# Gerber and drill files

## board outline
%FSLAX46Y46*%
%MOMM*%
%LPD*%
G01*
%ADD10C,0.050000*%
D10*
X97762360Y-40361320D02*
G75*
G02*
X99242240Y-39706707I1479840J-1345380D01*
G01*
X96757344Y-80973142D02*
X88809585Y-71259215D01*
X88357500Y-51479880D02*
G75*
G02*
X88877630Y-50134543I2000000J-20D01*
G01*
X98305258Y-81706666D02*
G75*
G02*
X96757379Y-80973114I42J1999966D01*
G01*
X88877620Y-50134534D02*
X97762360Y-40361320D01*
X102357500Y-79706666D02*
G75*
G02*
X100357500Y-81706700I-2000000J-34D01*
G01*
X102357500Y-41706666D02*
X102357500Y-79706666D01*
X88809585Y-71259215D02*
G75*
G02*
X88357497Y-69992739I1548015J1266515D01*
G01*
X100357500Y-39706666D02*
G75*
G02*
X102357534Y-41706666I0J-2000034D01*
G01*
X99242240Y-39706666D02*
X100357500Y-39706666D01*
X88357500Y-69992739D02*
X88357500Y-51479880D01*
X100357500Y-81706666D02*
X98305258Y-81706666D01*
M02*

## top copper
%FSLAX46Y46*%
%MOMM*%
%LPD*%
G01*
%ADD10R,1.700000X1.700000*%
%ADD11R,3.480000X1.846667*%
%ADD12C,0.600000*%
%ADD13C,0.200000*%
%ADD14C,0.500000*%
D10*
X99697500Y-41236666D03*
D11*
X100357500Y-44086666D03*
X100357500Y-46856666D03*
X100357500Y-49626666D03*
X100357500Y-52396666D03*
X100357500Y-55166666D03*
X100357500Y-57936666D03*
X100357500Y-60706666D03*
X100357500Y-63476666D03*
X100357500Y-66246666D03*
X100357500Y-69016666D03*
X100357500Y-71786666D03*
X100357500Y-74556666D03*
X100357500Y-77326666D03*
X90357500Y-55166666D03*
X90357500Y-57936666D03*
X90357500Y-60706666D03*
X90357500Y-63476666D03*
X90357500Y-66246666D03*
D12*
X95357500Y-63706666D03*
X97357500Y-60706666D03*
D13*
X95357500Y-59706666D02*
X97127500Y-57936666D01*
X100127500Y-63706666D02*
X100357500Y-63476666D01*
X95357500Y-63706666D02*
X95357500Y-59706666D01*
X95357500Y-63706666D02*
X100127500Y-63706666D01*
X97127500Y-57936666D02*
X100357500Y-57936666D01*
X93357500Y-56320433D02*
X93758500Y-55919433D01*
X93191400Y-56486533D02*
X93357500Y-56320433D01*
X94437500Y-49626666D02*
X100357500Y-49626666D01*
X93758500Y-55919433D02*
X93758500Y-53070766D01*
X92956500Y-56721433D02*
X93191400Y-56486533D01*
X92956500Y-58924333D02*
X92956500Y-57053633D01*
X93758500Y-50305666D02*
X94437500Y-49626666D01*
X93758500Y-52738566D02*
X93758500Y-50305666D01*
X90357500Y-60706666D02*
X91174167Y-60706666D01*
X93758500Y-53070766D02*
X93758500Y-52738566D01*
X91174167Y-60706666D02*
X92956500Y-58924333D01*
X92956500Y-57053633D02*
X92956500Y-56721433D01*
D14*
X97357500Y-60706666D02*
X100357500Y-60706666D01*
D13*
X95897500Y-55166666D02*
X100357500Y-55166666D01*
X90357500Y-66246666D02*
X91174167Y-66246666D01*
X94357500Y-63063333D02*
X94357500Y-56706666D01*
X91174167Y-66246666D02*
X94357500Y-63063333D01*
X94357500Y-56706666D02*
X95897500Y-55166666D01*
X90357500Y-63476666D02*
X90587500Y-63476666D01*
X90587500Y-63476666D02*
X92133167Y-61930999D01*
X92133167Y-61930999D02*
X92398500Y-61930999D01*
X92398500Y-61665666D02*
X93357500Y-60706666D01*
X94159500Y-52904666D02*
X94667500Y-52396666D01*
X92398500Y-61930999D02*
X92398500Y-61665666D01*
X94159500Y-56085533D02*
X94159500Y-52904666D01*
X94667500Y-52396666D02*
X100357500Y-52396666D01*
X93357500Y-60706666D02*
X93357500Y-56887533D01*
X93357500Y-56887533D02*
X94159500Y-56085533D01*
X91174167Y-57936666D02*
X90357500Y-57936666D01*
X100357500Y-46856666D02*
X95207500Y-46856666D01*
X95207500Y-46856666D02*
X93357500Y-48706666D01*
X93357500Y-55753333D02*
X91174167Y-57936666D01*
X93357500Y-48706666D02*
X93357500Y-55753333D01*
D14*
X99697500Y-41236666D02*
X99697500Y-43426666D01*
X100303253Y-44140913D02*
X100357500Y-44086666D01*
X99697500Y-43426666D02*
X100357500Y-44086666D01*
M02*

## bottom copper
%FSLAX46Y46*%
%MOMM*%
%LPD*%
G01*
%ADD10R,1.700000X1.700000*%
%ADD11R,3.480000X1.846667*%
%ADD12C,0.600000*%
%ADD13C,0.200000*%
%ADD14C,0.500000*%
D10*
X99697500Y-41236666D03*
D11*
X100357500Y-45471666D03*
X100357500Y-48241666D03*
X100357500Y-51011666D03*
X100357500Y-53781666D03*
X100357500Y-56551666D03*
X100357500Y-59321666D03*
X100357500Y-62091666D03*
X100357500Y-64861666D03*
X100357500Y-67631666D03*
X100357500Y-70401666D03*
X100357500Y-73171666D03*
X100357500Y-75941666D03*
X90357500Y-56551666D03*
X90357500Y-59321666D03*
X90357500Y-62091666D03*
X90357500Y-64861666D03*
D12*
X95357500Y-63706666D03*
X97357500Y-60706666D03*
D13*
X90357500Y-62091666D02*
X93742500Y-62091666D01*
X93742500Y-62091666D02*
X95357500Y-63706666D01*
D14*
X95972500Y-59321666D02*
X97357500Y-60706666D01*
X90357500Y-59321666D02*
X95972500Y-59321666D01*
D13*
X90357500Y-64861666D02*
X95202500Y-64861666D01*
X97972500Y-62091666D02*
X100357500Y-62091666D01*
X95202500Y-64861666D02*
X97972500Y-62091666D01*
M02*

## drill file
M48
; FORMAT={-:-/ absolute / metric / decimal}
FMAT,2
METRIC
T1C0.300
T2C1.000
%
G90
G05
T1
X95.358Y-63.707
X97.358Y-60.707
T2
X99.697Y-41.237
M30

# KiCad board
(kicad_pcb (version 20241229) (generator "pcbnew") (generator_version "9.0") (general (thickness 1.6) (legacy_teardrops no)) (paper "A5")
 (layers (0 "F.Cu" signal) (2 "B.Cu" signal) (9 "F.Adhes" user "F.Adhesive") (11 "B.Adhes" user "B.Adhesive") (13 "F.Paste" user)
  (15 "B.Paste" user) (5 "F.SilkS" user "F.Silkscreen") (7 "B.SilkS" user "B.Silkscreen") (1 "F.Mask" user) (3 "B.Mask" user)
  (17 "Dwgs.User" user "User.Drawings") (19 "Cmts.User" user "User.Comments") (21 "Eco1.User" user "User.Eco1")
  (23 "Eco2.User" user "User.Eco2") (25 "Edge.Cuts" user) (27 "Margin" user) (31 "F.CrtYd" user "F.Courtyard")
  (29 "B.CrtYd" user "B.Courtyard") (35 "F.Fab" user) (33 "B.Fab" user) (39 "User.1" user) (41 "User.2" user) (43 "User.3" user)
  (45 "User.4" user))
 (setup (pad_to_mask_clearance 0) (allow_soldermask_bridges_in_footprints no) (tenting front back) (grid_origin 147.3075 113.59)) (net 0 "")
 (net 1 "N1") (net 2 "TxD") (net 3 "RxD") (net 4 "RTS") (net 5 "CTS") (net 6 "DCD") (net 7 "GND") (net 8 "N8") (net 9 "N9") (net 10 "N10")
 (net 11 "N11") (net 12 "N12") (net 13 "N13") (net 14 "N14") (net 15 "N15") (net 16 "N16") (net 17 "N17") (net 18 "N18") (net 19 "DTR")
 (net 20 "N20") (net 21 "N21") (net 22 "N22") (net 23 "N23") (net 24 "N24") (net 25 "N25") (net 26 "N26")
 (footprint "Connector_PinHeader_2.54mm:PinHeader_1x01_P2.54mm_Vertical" (layer "F.Cu") (at 99.6975 41.236666)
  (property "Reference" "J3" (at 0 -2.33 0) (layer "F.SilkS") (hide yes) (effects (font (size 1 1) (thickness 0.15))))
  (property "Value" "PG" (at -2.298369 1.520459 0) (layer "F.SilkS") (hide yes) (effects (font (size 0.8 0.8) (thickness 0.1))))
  (pad "1" thru_hole rect (at 0 0) (size 1.7 1.7) (drill 1) (layers "*.Cu" "*.Mask") (remove_unused_layers no) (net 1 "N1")))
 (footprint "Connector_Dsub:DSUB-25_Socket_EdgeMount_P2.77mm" (layer "F.Cu") (at 100.3575 60.706666 90)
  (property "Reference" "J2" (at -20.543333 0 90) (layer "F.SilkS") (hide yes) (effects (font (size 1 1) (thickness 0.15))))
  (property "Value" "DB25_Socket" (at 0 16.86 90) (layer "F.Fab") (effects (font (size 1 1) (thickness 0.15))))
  (pad "1" smd rect (at 16.62 0 90) (size 1.846667 3.48) (layers "F.Cu" "F.Mask" "F.Paste") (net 1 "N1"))
  (pad "2" smd rect (at 13.85 0 90) (size 1.846667 3.48) (layers "F.Cu" "F.Mask" "F.Paste") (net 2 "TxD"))
  (pad "3" smd rect (at 11.08 0 90) (size 1.846667 3.48) (layers "F.Cu" "F.Mask" "F.Paste") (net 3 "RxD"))
  (pad "4" smd rect (at 8.31 0 90) (size 1.846667 3.48) (layers "F.Cu" "F.Mask" "F.Paste") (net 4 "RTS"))
  (pad "5" smd rect (at 5.54 0 90) (size 1.846667 3.48) (layers "F.Cu" "F.Mask" "F.Paste") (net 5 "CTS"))
  (pad "6" smd rect (at 2.77 0 90) (size 1.846667 3.48) (layers "F.Cu" "F.Mask" "F.Paste") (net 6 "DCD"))
  (pad "7" smd rect (at 0 0 90) (size 1.846667 3.48) (layers "F.Cu" "F.Mask" "F.Paste") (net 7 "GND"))
  (pad "8" smd rect (at -2.77 0 90) (size 1.846667 3.48) (layers "F.Cu" "F.Mask" "F.Paste") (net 6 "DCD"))
  (pad "9" smd rect (at -5.54 0 90) (size 1.846667 3.48) (layers "F.Cu" "F.Mask" "F.Paste") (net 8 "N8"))
  (pad "10" smd rect (at -8.31 0 90) (size 1.846667 3.48) (layers "F.Cu" "F.Mask" "F.Paste") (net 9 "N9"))
  (pad "11" smd rect (at -11.08 0 90) (size 1.846667 3.48) (layers "F.Cu" "F.Mask" "F.Paste") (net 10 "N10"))
  (pad "12" smd rect (at -13.85 0 90) (size 1.846667 3.48) (layers "F.Cu" "F.Mask" "F.Paste") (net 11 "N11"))
  (pad "13" smd rect (at -16.62 0 90) (size 1.846667 3.48) (layers "F.Cu" "F.Mask" "F.Paste") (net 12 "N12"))
  (pad "14" smd rect (at 15.235 0 90) (size 1.846667 3.48) (layers "B.Cu" "B.Mask" "B.Paste") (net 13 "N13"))
  (pad "15" smd rect (at 12.465 0 90) (size 1.846667 3.48) (layers "B.Cu" "B.Mask" "B.Paste") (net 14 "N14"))
  (pad "16" smd rect (at 9.695 0 90) (size 1.846667 3.48) (layers "B.Cu" "B.Mask" "B.Paste") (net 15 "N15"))
  (pad "17" smd rect (at 6.925 0 90) (size 1.846667 3.48) (layers "B.Cu" "B.Mask" "B.Paste") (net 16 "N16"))
  (pad "18" smd rect (at 4.155 0 90) (size 1.846667 3.48) (layers "B.Cu" "B.Mask" "B.Paste") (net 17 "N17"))
  (pad "19" smd rect (at 1.385 0 90) (size 1.846667 3.48) (layers "B.Cu" "B.Mask" "B.Paste") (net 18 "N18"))
  (pad "20" smd rect (at -1.385 0 90) (size 1.846667 3.48) (layers "B.Cu" "B.Mask" "B.Paste") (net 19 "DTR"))
  (pad "21" smd rect (at -4.155 0 90) (size 1.846667 3.48) (layers "B.Cu" "B.Mask" "B.Paste") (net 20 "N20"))
  (pad "22" smd rect (at -6.925 0 90) (size 1.846667 3.48) (layers "B.Cu" "B.Mask" "B.Paste") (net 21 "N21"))
  (pad "23" smd rect (at -9.695 0 90) (size 1.846667 3.48) (layers "B.Cu" "B.Mask" "B.Paste") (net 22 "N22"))
  (pad "24" smd rect (at -12.465 0 90) (size 1.846667 3.48) (layers "B.Cu" "B.Mask" "B.Paste") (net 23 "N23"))
  (pad "25" smd rect (at -15.235 0 90) (size 1.846667 3.48) (layers "B.Cu" "B.Mask" "B.Paste") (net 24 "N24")))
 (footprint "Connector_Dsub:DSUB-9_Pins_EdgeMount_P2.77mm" (layer "F.Cu") (at 90.3575 60.706666 -90)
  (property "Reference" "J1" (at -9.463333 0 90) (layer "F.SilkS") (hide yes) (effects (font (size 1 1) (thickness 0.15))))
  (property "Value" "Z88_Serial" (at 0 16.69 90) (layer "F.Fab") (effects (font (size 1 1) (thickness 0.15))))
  (pad "1" smd rect (at -5.54 0 270) (size 1.846667 3.48) (layers "F.Cu" "F.Mask" "F.Paste") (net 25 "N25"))
  (pad "2" smd rect (at -2.77 0 270) (size 1.846667 3.48) (layers "F.Cu" "F.Mask" "F.Paste") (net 2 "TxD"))
  (pad "3" smd rect (at 0 0 270) (size 1.846667 3.48) (layers "F.Cu" "F.Mask" "F.Paste") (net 3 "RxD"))
  (pad "4" smd rect (at 2.77 0 270) (size 1.846667 3.48) (layers "F.Cu" "F.Mask" "F.Paste") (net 4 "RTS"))
  (pad "5" smd rect (at 5.54 0 270) (size 1.846667 3.48) (layers "F.Cu" "F.Mask" "F.Paste") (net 5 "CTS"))
  (pad "6" smd rect (at -4.155 0 270) (size 1.846667 3.48) (layers "B.Cu" "B.Mask" "B.Paste") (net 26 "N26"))
  (pad "7" smd rect (at -1.385 0 270) (size 1.846667 3.48) (layers "B.Cu" "B.Mask" "B.Paste") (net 7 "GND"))
  (pad "8" smd rect (at 1.385 0 270) (size 1.846667 3.48) (layers "B.Cu" "B.Mask" "B.Paste") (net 6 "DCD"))
  (pad "9" smd rect (at 4.155 0 270) (size 1.846667 3.48) (layers "B.Cu" "B.Mask" "B.Paste") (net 19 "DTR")))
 (gr_arc (start 97.76236 40.36132) (mid 98.433133 39.877637) (end 99.24224 39.706666) (stroke (width 0.05) (type default))
  (layer "Edge.Cuts"))
 (gr_line (start 96.757344 80.973142) (end 88.809585 71.259215) (stroke (width 0.05) (type default)) (layer "Edge.Cuts"))
 (gr_arc (start 88.3575 51.47988) (mid 88.492056 50.758686) (end 88.87762 50.134534) (stroke (width 0.05) (type default))
  (layer "Edge.Cuts"))
 (gr_arc (start 98.305258 81.706666) (mid 97.448798 81.514006) (end 96.757344 80.973142) (stroke (width 0.05) (type default))
  (layer "Edge.Cuts"))
 (gr_line (start 88.87762 50.134534) (end 97.76236 40.36132) (stroke (width 0.05) (type default)) (layer "Edge.Cuts"))
 (gr_arc (start 102.3575 79.706666) (mid 101.771714 81.12088) (end 100.3575 81.706666) (stroke (width 0.05) (type default))
  (layer "Edge.Cuts"))
 (gr_line (start 102.3575 41.706666) (end 102.3575 79.706666) (stroke (width 0.05) (type default)) (layer "Edge.Cuts"))
 (gr_arc (start 88.809585 71.259215) (mid 88.473917 70.665111) (end 88.3575 69.992739) (stroke (width 0.05) (type default))
  (layer "Edge.Cuts"))
 (gr_arc (start 100.3575 39.706666) (mid 101.771714 40.292452) (end 102.3575 41.706666) (stroke (width 0.05) (type default))
  (layer "Edge.Cuts"))
 (gr_line (start 99.24224 39.706666) (end 100.3575 39.706666) (stroke (width 0.05) (type default)) (layer "Edge.Cuts"))
 (gr_line (start 88.3575 69.992739) (end 88.3575 51.47988) (stroke (width 0.05) (type default)) (layer "Edge.Cuts"))
 (gr_line (start 100.3575 81.706666) (end 98.305258 81.706666) (stroke (width 0.05) (type default)) (layer "Edge.Cuts"))
 (segment (start 95.3575 59.706666) (end 97.1275 57.936666) (width 0.2) (layer "F.Cu") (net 6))
 (segment (start 100.1275 63.706666) (end 100.3575 63.476666) (width 0.2) (layer "F.Cu") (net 6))
 (segment (start 95.3575 63.706666) (end 95.3575 59.706666) (width 0.2) (layer "F.Cu") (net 6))
 (segment (start 95.3575 63.706666) (end 100.1275 63.706666) (width 0.2) (layer "F.Cu") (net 6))
 (segment (start 97.1275 57.936666) (end 100.3575 57.936666) (width 0.2) (layer "F.Cu") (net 6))
 (via (at 95.3575 63.706666) (size 0.6) (drill 0.3) (layers "F.Cu" "B.Cu") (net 6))
 (segment (start 90.3575 62.091666) (end 93.7425 62.091666) (width 0.2) (layer "B.Cu") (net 6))
 (segment (start 93.7425 62.091666) (end 95.3575 63.706666) (width 0.2) (layer "B.Cu") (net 6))
 (segment (start 93.3575 56.320433) (end 93.7585 55.919433) (width 0.2) (layer "F.Cu") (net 3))
 (segment (start 93.1914 56.486533) (end 93.3575 56.320433) (width 0.2) (layer "F.Cu") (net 3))
 (segment (start 94.4375 49.626666) (end 100.3575 49.626666) (width 0.2) (layer "F.Cu") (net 3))
 (segment (start 93.7585 55.919433) (end 93.7585 53.070766) (width 0.2) (layer "F.Cu") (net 3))
 (segment (start 92.9565 56.721433) (end 93.1914 56.486533) (width 0.2) (layer "F.Cu") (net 3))
 (segment (start 92.9565 58.924333) (end 92.9565 57.053633) (width 0.2) (layer "F.Cu") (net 3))
 (segment (start 93.7585 50.305666) (end 94.4375 49.626666) (width 0.2) (layer "F.Cu") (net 3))
 (segment (start 93.7585 52.738566) (end 93.7585 50.305666) (width 0.2) (layer "F.Cu") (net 3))
 (segment (start 90.3575 60.706666) (end 91.174167 60.706666) (width 0.2) (layer "F.Cu") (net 3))
 (segment (start 93.7585 53.070766) (end 93.7585 52.738566) (width 0.2) (layer "F.Cu") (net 3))
 (segment (start 91.174167 60.706666) (end 92.9565 58.924333) (width 0.2) (layer "F.Cu") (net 3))
 (segment (start 92.9565 57.053633) (end 92.9565 56.721433) (width 0.2) (layer "F.Cu") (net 3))
 (segment (start 97.3575 60.706666) (end 100.3575 60.706666) (width 0.5) (layer "F.Cu") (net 7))
 (via (at 97.3575 60.706666) (size 0.6) (drill 0.3) (layers "F.Cu" "B.Cu") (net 7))
 (segment (start 95.9725 59.321666) (end 97.3575 60.706666) (width 0.5) (layer "B.Cu") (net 7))
 (segment (start 90.3575 59.321666) (end 95.9725 59.321666) (width 0.5) (layer "B.Cu") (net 7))
 (segment (start 95.8975 55.166666) (end 100.3575 55.166666) (width 0.2) (layer "F.Cu") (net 5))
 (segment (start 90.3575 66.246666) (end 91.174167 66.246666) (width 0.2) (layer "F.Cu") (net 5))
 (segment (start 94.3575 63.063333) (end 94.3575 56.706666) (width 0.2) (layer "F.Cu") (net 5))
 (segment (start 91.174167 66.246666) (end 94.3575 63.063333) (width 0.2) (layer "F.Cu") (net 5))
 (segment (start 94.3575 56.706666) (end 95.8975 55.166666) (width 0.2) (layer "F.Cu") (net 5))
 (segment (start 90.3575 64.861666) (end 95.2025 64.861666) (width 0.2) (layer "B.Cu") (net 19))
 (segment (start 97.9725 62.091666) (end 100.3575 62.091666) (width 0.2) (layer "B.Cu") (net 19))
 (segment (start 95.2025 64.861666) (end 97.9725 62.091666) (width 0.2) (layer "B.Cu") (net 19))
 (segment (start 90.3575 63.476666) (end 90.5875 63.476666) (width 0.2) (layer "F.Cu") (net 4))
 (segment (start 90.5875 63.476666) (end 92.133167 61.930999) (width 0.2) (layer "F.Cu") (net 4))
 (segment (start 92.133167 61.930999) (end 92.3985 61.930999) (width 0.2) (layer "F.Cu") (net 4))
 (segment (start 92.3985 61.665666) (end 93.3575 60.706666) (width 0.2) (layer "F.Cu") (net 4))
 (segment (start 94.1595 52.904666) (end 94.6675 52.396666) (width 0.2) (layer "F.Cu") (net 4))
 (segment (start 92.3985 61.930999) (end 92.3985 61.665666) (width 0.2) (layer "F.Cu") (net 4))
 (segment (start 94.1595 56.085533) (end 94.1595 52.904666) (width 0.2) (layer "F.Cu") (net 4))
 (segment (start 94.6675 52.396666) (end 100.3575 52.396666) (width 0.2) (layer "F.Cu") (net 4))
 (segment (start 93.3575 60.706666) (end 93.3575 56.887533) (width 0.2) (layer "F.Cu") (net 4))
 (segment (start 93.3575 56.887533) (end 94.1595 56.085533) (width 0.2) (layer "F.Cu") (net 4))
 (segment (start 91.174167 57.936666) (end 90.3575 57.936666) (width 0.2) (layer "F.Cu") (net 2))
 (segment (start 100.3575 46.856666) (end 95.2075 46.856666) (width 0.2) (layer "F.Cu") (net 2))
 (segment (start 95.2075 46.856666) (end 93.3575 48.706666) (width 0.2) (layer "F.Cu") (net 2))
 (segment (start 93.3575 55.753333) (end 91.174167 57.936666) (width 0.2) (layer "F.Cu") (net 2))
 (segment (start 93.3575 48.706666) (end 93.3575 55.753333) (width 0.2) (layer "F.Cu") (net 2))
 (segment (start 99.6975 41.236666) (end 99.6975 43.426666) (width 0.5) (layer "F.Cu") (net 1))
 (segment (start 100.303253 44.140913) (end 100.3575 44.086666) (width 0.5) (layer "F.Cu") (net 1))
 (segment (start 99.6975 43.426666) (end 100.3575 44.086666) (width 0.5) (layer "F.Cu") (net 1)))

